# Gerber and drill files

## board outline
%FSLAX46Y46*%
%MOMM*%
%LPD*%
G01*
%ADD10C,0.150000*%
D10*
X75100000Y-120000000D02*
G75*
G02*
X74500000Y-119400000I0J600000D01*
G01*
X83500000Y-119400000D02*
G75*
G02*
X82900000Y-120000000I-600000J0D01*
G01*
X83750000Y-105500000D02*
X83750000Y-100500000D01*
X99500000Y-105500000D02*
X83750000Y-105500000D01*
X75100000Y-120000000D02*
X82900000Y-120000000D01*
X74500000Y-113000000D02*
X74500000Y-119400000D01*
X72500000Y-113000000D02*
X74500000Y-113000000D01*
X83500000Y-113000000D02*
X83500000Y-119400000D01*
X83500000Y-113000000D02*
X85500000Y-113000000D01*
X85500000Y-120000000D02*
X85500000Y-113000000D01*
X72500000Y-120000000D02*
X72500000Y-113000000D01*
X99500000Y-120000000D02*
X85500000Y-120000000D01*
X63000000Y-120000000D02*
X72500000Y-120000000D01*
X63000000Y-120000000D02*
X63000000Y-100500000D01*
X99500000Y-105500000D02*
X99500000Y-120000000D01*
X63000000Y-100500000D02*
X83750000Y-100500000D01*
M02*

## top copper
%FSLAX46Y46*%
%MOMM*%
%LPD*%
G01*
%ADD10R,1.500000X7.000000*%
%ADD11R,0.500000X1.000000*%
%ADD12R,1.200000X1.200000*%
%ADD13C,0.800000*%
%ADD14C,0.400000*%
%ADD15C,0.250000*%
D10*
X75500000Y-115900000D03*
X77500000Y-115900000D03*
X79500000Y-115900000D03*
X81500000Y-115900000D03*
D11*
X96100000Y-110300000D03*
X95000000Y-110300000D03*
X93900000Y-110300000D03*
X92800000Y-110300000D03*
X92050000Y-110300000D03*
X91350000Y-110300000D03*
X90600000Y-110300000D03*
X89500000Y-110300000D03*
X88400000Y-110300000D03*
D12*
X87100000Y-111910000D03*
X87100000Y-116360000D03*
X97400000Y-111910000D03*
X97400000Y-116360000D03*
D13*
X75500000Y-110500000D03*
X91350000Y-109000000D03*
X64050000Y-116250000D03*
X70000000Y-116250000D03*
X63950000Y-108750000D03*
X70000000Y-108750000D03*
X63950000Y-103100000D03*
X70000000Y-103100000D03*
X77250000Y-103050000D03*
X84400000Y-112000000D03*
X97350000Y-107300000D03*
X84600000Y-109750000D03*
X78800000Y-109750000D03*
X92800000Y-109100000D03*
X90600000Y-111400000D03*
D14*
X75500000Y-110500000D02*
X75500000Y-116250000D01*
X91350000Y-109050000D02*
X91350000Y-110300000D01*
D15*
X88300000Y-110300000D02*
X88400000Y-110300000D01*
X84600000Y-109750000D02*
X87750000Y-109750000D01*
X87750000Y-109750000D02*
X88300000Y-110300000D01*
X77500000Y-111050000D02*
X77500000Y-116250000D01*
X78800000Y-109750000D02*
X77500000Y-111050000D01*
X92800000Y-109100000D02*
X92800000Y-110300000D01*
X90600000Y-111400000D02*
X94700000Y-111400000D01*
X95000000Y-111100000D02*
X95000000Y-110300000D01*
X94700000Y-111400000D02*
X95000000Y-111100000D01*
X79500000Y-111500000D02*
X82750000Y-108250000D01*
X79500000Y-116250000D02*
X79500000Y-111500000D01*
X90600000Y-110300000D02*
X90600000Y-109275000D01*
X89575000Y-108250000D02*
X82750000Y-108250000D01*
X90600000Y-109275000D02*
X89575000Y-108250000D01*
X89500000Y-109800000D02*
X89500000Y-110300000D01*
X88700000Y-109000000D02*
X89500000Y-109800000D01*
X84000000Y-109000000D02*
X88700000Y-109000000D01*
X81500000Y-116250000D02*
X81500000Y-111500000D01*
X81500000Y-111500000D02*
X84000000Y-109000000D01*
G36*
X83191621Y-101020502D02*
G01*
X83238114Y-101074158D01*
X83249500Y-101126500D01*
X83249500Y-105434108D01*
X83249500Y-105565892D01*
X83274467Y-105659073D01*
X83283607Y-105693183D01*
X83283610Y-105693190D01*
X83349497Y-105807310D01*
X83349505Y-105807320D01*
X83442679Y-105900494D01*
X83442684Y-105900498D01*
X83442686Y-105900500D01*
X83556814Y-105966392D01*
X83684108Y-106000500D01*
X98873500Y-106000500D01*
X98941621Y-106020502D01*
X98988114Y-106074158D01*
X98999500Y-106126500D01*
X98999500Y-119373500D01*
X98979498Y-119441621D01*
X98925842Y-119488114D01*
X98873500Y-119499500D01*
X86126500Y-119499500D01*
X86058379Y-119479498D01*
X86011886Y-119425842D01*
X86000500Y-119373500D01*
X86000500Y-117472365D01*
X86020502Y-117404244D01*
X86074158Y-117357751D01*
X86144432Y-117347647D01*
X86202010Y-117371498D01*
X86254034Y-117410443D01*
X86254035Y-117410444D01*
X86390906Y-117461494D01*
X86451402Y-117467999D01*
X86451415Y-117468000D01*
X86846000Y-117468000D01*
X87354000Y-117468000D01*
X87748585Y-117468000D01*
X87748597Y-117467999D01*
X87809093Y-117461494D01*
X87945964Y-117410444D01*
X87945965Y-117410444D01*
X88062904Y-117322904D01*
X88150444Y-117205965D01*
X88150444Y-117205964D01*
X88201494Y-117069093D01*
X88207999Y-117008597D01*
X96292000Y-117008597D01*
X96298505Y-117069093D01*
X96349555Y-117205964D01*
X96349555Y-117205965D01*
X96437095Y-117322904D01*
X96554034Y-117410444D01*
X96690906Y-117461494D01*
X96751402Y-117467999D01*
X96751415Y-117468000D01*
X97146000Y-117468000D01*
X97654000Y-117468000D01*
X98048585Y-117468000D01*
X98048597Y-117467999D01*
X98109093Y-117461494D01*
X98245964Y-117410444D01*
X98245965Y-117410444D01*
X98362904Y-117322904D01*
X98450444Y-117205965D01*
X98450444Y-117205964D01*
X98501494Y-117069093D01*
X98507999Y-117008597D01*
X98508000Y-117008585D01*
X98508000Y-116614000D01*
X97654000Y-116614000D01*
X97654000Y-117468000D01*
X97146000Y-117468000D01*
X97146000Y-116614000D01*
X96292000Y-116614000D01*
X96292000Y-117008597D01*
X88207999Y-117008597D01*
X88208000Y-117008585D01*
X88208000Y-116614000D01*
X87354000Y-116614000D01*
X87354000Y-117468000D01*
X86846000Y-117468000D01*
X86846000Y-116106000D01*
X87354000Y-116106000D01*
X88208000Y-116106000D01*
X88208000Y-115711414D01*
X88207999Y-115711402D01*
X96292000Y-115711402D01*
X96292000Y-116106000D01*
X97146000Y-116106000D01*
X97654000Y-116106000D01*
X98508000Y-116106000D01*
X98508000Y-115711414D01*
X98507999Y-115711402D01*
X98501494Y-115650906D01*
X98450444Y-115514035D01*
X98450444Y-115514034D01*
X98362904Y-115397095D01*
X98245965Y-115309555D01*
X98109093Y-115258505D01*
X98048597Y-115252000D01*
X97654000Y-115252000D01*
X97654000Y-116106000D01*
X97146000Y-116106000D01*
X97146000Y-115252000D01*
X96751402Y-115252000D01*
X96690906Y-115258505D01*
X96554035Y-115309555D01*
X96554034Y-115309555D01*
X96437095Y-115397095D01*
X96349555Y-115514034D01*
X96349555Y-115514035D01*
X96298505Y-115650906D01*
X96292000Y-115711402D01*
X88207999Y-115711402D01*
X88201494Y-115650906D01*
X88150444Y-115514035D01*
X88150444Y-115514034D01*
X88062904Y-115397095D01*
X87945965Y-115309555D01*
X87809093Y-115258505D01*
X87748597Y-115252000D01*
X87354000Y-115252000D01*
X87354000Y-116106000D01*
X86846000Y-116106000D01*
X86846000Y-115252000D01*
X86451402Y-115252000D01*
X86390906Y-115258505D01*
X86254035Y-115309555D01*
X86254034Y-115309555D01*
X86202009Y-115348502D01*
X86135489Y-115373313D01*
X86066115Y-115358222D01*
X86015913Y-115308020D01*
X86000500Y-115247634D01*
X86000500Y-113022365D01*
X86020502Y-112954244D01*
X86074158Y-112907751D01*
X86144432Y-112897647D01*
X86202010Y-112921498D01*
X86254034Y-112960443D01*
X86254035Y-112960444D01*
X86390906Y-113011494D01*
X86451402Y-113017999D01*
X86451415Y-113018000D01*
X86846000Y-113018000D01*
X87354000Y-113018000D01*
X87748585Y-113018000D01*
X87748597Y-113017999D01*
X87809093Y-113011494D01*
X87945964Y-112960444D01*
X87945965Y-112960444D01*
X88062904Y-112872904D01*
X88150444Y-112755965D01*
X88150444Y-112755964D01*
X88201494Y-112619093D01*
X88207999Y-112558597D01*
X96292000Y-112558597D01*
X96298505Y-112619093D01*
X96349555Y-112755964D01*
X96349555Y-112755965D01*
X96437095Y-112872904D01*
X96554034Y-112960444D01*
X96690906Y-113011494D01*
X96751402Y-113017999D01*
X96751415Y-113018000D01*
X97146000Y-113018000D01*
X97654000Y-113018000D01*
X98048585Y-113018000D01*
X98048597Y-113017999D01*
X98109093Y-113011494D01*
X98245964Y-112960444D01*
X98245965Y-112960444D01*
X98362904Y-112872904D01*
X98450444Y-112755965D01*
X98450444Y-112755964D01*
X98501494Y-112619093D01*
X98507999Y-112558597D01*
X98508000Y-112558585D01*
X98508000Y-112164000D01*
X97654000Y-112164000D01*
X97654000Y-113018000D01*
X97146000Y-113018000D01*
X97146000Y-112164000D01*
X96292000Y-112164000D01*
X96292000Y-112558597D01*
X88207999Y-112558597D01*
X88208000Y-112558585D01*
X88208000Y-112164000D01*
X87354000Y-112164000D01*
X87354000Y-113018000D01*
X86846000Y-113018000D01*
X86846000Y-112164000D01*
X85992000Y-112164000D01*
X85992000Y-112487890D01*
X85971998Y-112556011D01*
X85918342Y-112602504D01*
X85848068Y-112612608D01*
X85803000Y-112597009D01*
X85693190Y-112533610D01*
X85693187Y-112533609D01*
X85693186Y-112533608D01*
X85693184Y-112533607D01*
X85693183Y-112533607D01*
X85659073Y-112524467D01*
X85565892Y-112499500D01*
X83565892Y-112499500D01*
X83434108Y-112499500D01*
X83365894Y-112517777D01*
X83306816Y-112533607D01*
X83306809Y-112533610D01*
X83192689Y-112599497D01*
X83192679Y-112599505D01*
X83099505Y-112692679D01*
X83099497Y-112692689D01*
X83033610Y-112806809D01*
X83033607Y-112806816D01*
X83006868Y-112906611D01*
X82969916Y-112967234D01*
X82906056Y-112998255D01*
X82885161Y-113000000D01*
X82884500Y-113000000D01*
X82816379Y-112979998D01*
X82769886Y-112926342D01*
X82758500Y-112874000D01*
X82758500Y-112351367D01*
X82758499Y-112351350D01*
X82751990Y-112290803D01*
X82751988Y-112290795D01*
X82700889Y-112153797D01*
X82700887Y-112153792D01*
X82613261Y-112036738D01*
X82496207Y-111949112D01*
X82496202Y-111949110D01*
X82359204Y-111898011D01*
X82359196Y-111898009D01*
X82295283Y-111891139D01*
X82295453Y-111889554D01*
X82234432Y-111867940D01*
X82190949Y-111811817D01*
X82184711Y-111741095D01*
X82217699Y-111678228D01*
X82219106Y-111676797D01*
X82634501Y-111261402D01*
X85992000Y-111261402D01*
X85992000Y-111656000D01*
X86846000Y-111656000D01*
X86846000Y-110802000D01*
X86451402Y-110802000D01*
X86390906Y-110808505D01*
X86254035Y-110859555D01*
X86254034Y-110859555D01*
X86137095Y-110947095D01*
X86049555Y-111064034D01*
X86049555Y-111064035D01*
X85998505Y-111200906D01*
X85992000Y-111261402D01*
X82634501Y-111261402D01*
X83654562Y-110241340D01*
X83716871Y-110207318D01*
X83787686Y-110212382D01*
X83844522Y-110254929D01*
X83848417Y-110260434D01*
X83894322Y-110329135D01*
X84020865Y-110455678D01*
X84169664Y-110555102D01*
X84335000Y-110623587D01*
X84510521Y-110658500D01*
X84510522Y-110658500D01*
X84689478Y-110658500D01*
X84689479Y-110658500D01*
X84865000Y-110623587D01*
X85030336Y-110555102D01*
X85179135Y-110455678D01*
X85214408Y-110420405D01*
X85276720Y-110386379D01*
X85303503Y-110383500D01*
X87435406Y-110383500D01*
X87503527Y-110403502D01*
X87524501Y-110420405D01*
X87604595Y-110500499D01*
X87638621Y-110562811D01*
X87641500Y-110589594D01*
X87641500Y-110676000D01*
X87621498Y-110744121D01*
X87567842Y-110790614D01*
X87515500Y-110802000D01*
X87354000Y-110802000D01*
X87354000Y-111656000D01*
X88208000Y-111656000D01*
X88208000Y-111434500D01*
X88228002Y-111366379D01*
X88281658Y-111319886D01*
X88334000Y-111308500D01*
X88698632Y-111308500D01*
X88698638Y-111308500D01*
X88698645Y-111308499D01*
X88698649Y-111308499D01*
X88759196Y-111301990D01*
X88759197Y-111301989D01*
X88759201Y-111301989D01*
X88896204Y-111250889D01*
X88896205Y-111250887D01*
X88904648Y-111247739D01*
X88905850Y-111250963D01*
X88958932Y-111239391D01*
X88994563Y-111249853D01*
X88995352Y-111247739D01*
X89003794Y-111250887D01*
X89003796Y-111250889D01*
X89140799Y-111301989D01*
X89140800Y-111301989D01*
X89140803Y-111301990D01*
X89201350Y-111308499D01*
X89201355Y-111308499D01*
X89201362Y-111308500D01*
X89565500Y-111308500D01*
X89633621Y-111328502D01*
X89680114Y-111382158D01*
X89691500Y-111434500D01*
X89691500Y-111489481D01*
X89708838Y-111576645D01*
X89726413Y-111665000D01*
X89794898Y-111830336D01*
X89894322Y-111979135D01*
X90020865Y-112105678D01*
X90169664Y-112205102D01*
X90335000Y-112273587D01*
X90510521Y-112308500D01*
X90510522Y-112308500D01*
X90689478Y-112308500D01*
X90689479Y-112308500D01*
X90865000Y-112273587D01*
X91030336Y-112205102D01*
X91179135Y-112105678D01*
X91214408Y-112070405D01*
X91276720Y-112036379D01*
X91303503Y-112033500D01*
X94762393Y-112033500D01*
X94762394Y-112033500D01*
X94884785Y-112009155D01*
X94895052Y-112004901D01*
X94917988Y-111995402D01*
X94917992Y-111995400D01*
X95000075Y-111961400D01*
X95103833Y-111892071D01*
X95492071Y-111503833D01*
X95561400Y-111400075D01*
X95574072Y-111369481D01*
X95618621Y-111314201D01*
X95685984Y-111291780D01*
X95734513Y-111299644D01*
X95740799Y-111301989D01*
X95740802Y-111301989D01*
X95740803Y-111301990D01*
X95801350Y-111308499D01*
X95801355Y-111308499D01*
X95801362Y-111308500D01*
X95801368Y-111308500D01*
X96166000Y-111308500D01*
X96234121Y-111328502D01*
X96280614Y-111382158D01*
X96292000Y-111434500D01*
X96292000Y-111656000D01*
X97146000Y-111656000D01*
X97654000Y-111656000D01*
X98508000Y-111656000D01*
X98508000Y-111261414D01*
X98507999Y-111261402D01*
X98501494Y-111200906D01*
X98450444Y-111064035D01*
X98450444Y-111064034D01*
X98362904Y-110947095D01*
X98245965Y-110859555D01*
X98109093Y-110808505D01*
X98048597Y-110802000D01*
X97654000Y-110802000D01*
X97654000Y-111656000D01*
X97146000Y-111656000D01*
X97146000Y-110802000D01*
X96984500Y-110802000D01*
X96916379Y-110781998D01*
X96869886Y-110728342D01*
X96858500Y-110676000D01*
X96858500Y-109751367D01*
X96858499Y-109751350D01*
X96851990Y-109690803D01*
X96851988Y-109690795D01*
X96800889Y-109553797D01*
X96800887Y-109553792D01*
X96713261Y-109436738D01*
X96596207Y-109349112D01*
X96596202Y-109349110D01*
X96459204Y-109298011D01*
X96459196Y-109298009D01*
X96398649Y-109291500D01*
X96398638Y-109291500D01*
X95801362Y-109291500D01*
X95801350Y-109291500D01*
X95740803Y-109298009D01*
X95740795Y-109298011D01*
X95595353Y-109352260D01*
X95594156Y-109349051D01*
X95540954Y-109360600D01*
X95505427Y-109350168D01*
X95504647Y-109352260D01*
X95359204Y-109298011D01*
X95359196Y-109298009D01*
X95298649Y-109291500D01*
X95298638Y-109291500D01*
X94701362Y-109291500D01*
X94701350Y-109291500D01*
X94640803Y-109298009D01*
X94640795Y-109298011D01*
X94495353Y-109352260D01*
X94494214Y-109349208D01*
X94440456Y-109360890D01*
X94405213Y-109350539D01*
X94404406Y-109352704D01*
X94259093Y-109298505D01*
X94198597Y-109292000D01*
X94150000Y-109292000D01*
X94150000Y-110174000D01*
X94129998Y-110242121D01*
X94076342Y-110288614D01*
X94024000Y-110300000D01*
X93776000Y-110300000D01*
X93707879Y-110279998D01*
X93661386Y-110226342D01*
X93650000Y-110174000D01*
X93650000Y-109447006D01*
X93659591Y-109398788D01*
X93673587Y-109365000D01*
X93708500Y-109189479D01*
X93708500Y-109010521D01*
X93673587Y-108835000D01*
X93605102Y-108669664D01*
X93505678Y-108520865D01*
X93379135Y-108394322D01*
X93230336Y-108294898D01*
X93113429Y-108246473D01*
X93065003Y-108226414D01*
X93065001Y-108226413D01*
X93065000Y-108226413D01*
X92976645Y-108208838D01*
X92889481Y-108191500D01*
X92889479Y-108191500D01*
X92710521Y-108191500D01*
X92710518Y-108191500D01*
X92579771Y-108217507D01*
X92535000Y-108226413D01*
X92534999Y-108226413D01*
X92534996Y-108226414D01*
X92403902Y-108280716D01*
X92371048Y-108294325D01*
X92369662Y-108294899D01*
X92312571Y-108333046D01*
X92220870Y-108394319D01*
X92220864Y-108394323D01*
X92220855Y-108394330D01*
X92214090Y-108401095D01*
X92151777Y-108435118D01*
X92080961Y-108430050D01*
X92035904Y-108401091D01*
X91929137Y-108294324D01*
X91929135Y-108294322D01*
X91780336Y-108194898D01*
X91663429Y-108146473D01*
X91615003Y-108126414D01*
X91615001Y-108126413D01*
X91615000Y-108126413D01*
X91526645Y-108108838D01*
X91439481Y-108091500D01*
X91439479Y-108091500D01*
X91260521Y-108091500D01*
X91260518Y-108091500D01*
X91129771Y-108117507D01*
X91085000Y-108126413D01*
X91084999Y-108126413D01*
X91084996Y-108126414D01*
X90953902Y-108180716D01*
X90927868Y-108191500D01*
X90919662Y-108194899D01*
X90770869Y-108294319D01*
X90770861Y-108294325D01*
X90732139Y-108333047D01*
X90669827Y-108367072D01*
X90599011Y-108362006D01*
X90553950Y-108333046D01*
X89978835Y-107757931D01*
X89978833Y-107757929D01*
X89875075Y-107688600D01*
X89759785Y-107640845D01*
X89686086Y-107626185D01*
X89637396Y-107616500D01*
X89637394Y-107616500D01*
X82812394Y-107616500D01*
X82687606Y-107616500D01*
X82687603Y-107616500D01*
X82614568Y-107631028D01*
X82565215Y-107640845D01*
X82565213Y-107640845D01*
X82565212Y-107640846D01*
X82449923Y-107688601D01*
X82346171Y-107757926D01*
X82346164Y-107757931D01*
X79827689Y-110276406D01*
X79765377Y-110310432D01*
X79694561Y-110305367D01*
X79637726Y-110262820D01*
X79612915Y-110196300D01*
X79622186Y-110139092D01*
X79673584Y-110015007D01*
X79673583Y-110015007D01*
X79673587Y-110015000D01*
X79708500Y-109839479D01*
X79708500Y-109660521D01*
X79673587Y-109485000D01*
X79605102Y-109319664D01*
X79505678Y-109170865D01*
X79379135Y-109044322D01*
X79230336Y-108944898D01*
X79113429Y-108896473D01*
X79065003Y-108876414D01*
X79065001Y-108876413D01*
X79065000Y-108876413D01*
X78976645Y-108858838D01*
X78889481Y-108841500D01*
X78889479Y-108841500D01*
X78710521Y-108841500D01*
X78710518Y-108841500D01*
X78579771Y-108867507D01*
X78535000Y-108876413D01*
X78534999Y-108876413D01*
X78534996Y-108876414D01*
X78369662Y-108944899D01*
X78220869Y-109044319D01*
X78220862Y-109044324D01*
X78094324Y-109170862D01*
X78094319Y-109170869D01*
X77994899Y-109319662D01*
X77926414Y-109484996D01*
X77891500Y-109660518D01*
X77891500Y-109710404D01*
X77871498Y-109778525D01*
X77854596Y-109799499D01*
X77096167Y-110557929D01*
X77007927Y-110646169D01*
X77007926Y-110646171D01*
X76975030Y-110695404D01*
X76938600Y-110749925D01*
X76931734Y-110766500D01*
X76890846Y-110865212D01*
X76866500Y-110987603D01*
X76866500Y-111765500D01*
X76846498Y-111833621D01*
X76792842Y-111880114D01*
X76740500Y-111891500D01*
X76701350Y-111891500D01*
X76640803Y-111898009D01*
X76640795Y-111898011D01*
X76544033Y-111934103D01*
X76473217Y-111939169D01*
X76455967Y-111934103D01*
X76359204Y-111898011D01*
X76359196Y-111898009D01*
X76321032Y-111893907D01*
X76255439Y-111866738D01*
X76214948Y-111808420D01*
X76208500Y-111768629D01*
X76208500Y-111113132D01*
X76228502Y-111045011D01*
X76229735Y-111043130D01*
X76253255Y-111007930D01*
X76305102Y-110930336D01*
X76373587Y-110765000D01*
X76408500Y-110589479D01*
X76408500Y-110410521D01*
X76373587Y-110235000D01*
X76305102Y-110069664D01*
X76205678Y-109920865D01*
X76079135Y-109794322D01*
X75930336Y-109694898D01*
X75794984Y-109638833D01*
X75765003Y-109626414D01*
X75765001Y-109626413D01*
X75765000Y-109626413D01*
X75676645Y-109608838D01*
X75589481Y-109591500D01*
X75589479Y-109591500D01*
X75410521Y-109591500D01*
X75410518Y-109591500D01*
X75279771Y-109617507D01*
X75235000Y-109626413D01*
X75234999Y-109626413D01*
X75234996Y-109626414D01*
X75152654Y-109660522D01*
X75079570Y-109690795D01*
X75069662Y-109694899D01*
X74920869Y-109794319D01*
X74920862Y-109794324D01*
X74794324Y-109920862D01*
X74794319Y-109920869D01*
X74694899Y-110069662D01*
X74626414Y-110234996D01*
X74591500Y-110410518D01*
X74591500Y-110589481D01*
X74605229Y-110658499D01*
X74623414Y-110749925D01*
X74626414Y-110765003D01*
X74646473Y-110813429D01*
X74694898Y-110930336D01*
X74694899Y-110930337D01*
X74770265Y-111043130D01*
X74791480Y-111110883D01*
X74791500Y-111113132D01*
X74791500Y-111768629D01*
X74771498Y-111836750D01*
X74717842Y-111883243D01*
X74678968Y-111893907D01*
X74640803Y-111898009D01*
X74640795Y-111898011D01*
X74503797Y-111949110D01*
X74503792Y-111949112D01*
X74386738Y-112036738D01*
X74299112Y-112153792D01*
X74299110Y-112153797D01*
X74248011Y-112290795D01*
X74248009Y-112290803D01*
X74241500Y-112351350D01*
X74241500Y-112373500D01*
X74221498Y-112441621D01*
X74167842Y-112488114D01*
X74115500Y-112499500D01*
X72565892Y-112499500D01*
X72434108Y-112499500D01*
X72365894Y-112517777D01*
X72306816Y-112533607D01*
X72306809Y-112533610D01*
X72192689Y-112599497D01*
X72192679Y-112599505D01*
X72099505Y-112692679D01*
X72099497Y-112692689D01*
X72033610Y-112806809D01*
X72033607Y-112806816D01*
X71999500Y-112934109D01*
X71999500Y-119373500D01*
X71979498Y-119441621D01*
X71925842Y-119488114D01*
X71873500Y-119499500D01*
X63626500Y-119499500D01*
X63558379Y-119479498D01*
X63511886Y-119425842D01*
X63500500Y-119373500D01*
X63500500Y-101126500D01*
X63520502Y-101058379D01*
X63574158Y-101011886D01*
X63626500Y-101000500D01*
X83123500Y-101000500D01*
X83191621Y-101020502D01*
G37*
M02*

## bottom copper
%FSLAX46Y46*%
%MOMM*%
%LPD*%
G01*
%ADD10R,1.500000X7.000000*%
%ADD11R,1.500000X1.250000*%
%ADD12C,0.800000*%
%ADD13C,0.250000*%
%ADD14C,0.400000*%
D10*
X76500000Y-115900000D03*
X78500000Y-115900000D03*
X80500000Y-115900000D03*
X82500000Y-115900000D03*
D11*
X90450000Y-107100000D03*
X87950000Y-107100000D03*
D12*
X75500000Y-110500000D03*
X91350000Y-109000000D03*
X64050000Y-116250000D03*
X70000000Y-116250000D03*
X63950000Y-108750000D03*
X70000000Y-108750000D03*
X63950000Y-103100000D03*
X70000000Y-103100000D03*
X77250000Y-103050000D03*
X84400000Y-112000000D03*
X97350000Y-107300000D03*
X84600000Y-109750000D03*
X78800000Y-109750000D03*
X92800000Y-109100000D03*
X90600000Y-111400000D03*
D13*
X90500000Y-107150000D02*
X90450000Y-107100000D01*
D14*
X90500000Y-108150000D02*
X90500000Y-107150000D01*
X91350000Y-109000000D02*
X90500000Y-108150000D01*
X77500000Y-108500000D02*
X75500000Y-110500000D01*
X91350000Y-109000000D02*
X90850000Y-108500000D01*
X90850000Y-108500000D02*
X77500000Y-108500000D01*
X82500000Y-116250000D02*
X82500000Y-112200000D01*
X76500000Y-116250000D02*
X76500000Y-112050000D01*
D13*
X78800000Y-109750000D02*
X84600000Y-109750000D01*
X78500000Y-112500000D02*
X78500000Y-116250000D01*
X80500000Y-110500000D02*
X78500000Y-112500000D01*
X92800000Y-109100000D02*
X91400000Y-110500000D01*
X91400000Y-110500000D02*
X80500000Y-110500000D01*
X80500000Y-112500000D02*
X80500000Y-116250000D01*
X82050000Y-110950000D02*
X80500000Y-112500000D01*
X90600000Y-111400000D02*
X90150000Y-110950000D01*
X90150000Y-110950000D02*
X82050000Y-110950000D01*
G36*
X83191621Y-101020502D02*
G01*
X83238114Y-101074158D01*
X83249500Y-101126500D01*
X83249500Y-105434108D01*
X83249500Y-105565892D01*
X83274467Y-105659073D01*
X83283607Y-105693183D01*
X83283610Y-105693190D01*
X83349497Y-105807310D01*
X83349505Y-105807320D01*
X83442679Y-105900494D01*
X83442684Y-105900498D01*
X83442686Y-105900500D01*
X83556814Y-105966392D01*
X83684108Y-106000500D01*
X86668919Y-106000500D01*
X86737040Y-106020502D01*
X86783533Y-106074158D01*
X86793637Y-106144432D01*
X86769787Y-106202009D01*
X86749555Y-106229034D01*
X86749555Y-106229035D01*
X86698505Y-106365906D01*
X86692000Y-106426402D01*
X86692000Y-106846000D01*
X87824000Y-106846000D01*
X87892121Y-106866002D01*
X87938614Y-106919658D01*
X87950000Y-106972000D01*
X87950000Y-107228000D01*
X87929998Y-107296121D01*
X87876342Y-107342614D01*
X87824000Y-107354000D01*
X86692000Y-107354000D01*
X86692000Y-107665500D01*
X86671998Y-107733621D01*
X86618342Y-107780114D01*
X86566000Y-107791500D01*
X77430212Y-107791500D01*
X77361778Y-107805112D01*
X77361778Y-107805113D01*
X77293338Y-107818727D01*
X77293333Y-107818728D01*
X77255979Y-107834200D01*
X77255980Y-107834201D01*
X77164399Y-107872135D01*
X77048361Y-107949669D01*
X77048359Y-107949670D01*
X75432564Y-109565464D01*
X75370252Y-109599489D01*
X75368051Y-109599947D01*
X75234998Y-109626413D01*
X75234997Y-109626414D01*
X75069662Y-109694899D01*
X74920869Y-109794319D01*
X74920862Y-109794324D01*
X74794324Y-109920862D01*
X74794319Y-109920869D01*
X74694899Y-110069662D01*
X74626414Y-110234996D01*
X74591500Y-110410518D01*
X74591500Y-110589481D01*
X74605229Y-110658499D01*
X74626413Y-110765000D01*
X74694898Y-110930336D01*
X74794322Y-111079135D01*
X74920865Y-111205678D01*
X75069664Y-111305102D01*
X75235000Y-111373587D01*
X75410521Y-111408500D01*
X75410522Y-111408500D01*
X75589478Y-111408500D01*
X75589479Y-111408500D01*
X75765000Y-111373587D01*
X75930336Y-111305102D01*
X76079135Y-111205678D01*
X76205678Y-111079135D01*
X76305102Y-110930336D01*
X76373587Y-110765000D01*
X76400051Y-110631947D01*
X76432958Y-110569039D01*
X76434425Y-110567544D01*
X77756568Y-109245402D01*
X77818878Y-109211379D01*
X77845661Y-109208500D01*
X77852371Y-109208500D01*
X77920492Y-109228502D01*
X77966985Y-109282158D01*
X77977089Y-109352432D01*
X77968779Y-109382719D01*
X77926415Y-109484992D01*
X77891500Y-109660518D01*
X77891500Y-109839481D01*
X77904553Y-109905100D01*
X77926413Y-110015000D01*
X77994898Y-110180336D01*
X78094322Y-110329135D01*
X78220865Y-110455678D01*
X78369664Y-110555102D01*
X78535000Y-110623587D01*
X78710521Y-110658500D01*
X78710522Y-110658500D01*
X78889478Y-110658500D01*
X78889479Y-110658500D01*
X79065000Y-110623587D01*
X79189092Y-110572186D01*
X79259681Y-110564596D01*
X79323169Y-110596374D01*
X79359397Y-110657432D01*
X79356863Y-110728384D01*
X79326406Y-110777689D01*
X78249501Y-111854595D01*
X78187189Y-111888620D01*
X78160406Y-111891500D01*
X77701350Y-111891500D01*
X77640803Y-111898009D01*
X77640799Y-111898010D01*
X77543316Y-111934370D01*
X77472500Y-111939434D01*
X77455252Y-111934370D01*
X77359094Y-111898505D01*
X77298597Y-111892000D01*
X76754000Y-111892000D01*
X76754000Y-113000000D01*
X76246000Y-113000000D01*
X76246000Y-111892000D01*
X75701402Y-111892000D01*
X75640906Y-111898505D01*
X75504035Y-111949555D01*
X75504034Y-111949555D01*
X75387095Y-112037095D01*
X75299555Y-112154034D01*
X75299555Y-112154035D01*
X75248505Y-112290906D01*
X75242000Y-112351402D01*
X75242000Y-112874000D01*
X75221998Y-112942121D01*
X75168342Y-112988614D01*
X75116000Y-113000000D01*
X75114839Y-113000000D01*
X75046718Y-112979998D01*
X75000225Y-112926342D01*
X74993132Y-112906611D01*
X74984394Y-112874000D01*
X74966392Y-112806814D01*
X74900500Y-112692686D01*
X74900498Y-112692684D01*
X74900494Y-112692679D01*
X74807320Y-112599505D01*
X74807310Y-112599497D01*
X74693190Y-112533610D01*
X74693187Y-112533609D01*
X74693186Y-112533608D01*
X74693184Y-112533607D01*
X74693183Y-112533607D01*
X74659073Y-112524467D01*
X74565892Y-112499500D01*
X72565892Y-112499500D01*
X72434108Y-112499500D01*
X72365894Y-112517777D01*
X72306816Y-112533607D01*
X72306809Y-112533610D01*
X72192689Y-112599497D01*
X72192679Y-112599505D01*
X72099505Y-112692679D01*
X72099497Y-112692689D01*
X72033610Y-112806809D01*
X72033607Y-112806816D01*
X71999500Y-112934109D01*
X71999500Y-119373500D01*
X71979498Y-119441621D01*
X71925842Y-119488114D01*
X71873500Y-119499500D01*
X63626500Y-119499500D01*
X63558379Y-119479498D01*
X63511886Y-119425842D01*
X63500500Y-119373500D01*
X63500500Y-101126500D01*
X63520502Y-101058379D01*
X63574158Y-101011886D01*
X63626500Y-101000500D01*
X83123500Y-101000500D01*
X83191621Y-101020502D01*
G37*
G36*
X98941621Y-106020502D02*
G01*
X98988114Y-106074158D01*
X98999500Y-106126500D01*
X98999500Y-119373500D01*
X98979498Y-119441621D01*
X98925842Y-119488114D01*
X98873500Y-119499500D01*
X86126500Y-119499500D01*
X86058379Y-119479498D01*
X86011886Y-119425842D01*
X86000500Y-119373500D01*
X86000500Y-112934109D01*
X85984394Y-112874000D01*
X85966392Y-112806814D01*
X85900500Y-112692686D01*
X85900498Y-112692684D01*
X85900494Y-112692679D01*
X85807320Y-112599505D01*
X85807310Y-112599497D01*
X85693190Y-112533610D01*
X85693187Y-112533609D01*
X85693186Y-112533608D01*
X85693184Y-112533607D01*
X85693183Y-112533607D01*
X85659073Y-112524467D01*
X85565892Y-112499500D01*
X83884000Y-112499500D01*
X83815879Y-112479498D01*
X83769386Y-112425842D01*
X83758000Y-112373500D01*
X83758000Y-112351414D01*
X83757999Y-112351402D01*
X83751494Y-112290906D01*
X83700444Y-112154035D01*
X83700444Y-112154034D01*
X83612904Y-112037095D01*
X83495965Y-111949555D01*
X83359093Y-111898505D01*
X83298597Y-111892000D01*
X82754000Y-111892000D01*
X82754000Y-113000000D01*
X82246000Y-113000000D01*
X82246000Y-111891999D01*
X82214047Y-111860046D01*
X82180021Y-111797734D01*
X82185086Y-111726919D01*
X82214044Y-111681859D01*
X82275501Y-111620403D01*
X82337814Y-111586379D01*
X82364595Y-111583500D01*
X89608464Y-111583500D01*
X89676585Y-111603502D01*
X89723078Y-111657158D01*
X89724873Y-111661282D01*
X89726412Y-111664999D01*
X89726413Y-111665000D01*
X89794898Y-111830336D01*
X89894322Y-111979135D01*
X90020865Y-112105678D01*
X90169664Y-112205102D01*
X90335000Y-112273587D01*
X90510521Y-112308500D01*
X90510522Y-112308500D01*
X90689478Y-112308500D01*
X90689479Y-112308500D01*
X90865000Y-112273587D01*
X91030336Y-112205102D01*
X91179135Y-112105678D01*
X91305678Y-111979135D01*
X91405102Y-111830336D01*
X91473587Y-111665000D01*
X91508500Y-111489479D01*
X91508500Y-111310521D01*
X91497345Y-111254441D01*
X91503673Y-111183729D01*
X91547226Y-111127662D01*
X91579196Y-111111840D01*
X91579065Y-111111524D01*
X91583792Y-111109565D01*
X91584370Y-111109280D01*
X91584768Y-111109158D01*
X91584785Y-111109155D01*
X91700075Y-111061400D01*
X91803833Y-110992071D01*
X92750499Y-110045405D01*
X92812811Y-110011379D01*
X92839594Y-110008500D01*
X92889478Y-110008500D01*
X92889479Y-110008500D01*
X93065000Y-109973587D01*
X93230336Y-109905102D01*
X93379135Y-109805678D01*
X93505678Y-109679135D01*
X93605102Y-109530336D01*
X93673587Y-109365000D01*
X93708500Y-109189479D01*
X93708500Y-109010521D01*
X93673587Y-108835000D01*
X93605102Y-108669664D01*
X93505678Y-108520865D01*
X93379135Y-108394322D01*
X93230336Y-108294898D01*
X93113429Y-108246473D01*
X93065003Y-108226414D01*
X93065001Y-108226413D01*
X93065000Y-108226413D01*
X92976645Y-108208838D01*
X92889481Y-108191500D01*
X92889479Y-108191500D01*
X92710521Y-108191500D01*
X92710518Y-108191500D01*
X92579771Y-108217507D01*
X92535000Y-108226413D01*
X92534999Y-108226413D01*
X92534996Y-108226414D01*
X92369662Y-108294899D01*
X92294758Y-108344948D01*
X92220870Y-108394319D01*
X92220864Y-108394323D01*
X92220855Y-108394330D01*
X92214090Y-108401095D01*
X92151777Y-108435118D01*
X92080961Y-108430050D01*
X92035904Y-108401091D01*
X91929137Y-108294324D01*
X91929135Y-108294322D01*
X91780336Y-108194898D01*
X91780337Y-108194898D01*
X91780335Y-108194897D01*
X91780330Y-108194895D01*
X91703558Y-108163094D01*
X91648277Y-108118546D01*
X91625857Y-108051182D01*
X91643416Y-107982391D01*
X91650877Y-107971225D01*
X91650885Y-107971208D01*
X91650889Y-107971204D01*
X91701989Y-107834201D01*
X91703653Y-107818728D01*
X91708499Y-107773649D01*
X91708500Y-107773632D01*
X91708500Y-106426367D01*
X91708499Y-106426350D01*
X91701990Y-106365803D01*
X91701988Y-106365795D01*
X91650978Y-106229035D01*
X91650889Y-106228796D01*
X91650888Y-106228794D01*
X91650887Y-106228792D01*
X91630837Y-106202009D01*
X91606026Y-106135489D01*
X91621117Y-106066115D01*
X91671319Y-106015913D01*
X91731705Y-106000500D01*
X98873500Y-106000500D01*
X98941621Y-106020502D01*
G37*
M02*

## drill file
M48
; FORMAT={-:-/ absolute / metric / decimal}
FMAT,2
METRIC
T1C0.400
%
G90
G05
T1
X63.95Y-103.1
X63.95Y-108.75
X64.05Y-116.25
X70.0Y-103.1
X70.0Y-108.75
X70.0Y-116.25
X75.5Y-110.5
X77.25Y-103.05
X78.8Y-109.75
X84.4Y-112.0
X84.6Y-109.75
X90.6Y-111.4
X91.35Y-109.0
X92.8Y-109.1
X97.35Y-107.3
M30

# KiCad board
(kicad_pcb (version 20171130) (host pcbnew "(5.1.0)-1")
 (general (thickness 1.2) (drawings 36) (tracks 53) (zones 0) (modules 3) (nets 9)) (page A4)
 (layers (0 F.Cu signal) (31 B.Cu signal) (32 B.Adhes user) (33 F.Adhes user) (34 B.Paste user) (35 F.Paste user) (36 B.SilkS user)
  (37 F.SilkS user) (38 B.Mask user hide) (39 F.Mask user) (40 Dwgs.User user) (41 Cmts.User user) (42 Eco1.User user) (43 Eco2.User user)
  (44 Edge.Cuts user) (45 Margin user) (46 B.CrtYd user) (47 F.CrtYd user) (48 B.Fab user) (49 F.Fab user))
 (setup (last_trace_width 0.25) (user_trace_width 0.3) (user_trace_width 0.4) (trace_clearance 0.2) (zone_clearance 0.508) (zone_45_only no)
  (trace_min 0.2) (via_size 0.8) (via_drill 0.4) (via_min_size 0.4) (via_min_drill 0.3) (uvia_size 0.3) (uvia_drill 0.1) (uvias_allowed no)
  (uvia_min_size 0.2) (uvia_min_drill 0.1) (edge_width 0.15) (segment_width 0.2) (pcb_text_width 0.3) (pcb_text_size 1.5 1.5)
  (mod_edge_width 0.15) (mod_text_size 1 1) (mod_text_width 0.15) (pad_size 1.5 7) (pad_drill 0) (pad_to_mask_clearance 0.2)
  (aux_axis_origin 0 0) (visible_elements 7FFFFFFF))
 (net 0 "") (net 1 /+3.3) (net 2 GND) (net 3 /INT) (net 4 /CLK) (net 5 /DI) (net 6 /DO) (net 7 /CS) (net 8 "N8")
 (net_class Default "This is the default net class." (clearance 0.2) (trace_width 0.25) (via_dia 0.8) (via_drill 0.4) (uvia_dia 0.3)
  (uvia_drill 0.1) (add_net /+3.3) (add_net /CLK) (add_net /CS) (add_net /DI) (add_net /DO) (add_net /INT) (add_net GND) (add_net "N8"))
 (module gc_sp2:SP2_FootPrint (layer F.Cu) (at 75.5 115.9)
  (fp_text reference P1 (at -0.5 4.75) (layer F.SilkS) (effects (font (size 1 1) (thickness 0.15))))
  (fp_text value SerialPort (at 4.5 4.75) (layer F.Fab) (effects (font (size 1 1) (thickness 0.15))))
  (pad 1 smd rect (at 0 0) (size 1.5 7) (layers F.Cu F.Paste F.Mask) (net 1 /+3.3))
  (pad 2 smd rect (at 1 0) (size 1.5 7) (layers B.Cu B.Paste B.Mask) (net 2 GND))
  (pad 3 smd rect (at 2 0) (size 1.5 7) (layers F.Cu F.Paste F.Mask) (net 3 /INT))
  (pad 4 smd rect (at 3 0) (size 1.5 7) (layers B.Cu B.Adhes B.Mask) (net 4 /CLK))
  (pad 5 smd rect (at 4 0) (size 1.5 7) (layers F.Cu F.Paste F.Mask) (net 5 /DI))
  (pad 6 smd rect (at 5 0) (size 1.5 7) (layers B.Cu B.Paste B.Mask) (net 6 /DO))
  (pad 7 smd rect (at 6 0) (size 1.5 7) (layers F.Cu F.Paste F.Mask) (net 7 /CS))
  (pad 8 smd rect (at 7 0) (size 1.5 7) (layers B.Cu B.Paste B.Mask) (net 2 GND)))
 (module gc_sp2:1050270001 (layer F.Cu) (at 96.1 110.3 180)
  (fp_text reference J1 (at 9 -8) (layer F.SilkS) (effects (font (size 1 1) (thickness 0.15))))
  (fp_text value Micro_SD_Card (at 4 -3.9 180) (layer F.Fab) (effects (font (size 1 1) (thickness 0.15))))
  (pad 8 smd rect (at 0 0 180) (size 0.5 1) (layers F.Cu F.Paste F.Mask) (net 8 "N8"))
  (pad 7 smd rect (at 1.1 0 180) (size 0.5 1) (layers F.Cu F.Paste F.Mask) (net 6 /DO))
  (pad 6 smd rect (at 2.2 0 180) (size 0.5 1) (layers F.Cu F.Paste F.Mask) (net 2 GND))
  (pad 5 smd rect (at 3.3 0 180) (size 0.5 1) (layers F.Cu F.Paste F.Mask) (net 4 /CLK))
  (pad "" smd rect (at 4.05 0 180) (size 0.5 1) (layers F.Cu F.Paste F.Mask))
  (pad 4 smd rect (at 4.75 0 180) (size 0.5 1) (layers F.Cu F.Paste F.Mask) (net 1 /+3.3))
  (pad 3 smd rect (at 5.5 0 180) (size 0.5 1) (layers F.Cu F.Paste F.Mask) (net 5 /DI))
  (pad 2 smd rect (at 6.6 0 180) (size 0.5 1) (layers F.Cu F.Paste F.Mask) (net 7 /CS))
  (pad 1 smd rect (at 7.7 0 180) (size 0.5 1) (layers F.Cu F.Paste F.Mask) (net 3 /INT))
  (pad 9 smd rect (at 9 -1.61 180) (size 1.2 1.2) (layers F.Cu F.Paste F.Mask) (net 2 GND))
  (pad 9 smd rect (at 9 -6.06 180) (size 1.2 1.2) (layers F.Cu F.Paste F.Mask) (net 2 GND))
  (pad 9 smd rect (at -1.3 -1.61 180) (size 1.2 1.2) (layers F.Cu F.Paste F.Mask) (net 2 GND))
  (pad 9 smd rect (at -1.3 -6.06 180) (size 1.2 1.2) (layers F.Cu F.Paste F.Mask) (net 2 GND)))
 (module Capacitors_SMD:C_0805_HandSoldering (layer B.Cu) (at 89.2 107.1 180)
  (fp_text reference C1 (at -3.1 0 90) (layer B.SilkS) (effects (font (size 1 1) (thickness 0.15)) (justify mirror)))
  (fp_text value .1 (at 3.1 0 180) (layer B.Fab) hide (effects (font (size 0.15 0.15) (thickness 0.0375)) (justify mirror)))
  (pad 1 smd rect (at -1.25 0 180) (size 1.5 1.25) (layers B.Cu B.Paste B.Mask) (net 1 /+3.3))
  (pad 2 smd rect (at 1.25 0 180) (size 1.5 1.25) (layers B.Cu B.Paste B.Mask) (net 2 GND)))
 (gr_arc (start 75.1 119.4) (end 74.5 119.4) (angle -90) (layer Edge.Cuts) (width 0.15))
 (gr_arc (start 82.9 119.4) (end 82.9 120) (angle -90) (layer Edge.Cuts) (width 0.15))
 (gr_line (start 83.75 105.5) (end 83.75 100.5) (layer Edge.Cuts) (width 0.15))
 (gr_line (start 99.5 105.5) (end 83.75 105.5) (layer Edge.Cuts) (width 0.15))
 (gr_line (start 75.1 120) (end 82.9 120) (layer Edge.Cuts) (width 0.15))
 (gr_line (start 74.5 113) (end 74.5 119.4) (layer Edge.Cuts) (width 0.15))
 (gr_line (start 72.5 113) (end 74.5 113) (layer Edge.Cuts) (width 0.15))
 (gr_line (start 83.5 113) (end 83.5 119.4) (layer Edge.Cuts) (width 0.15))
 (gr_line (start 83.5 113) (end 85.5 113) (layer Edge.Cuts) (width 0.15))
 (gr_line (start 85.5 120) (end 85.5 113) (layer Edge.Cuts) (width 0.15))
 (gr_line (start 72.5 120) (end 72.5 113) (layer Edge.Cuts) (width 0.15))
 (gr_line (start 99.5 120) (end 85.5 120) (layer Edge.Cuts) (width 0.15))
 (gr_line (start 63 120) (end 72.5 120) (layer Edge.Cuts) (width 0.15))
 (gr_line (start 63 120) (end 63 100.5) (layer Edge.Cuts) (width 0.15))
 (gr_line (start 99.5 105.5) (end 99.5 120) (layer Edge.Cuts) (width 0.15))
 (gr_line (start 63 100.5) (end 83.75 100.5) (layer Edge.Cuts) (width 0.15))
 (via (at 75.5 110.5) (size 0.8) (drill 0.4) (layers F.Cu B.Cu) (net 1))
 (segment (start 75.5 110.5) (end 75.5 116.25) (width 0.4) (layer F.Cu) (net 1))
 (segment (start 90.5 107.15) (end 90.45 107.1) (width 0.25) (layer B.Cu) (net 1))
 (segment (start 91.35 109.05) (end 91.35 110.3) (width 0.4) (layer F.Cu) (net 1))
 (via (at 91.35 109) (size 0.8) (drill 0.4) (layers F.Cu B.Cu) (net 1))
 (segment (start 90.5 108.15) (end 90.5 107.15) (width 0.4) (layer B.Cu) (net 1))
 (segment (start 91.35 109) (end 90.5 108.15) (width 0.4) (layer B.Cu) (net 1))
 (segment (start 77.5 108.5) (end 75.5 110.5) (width 0.4) (layer B.Cu) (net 1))
 (segment (start 91.35 109) (end 90.85 108.5) (width 0.4) (layer B.Cu) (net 1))
 (segment (start 90.85 108.5) (end 77.5 108.5) (width 0.4) (layer B.Cu) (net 1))
 (via (at 64.05 116.25) (size 0.8) (drill 0.4) (layers F.Cu B.Cu) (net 2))
 (via (at 70 116.25) (size 0.8) (drill 0.4) (layers F.Cu B.Cu) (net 2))
 (via (at 63.95 108.75) (size 0.8) (drill 0.4) (layers F.Cu B.Cu) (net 2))
 (via (at 70 108.75) (size 0.8) (drill 0.4) (layers F.Cu B.Cu) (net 2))
 (via (at 63.95 103.1) (size 0.8) (drill 0.4) (layers F.Cu B.Cu) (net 2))
 (via (at 70 103.1) (size 0.8) (drill 0.4) (layers F.Cu B.Cu) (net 2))
 (via (at 77.25 103.05) (size 0.8) (drill 0.4) (layers F.Cu B.Cu) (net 2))
 (via (at 84.4 112) (size 0.8) (drill 0.4) (layers F.Cu B.Cu) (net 2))
 (via (at 97.35 107.3) (size 0.8) (drill 0.4) (layers F.Cu B.Cu) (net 2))
 (segment (start 82.5 116.25) (end 82.5 112.2) (width 0.4) (layer B.Cu) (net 2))
 (segment (start 76.5 116.25) (end 76.5 112.05) (width 0.4) (layer B.Cu) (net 2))
 (via (at 84.6 109.75) (size 0.8) (drill 0.4) (layers F.Cu B.Cu) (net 3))
 (segment (start 88.3 110.3) (end 88.4 110.3) (width 0.25) (layer F.Cu) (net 3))
 (segment (start 84.6 109.75) (end 87.75 109.75) (width 0.25) (layer F.Cu) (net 3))
 (segment (start 87.75 109.75) (end 88.3 110.3) (width 0.25) (layer F.Cu) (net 3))
 (via (at 78.8 109.75) (size 0.8) (drill 0.4) (layers F.Cu B.Cu) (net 3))
 (segment (start 78.8 109.75) (end 84.6 109.75) (width 0.25) (layer B.Cu) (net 3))
 (segment (start 77.5 111.05) (end 77.5 116.25) (width 0.25) (layer F.Cu) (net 3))
 (segment (start 78.8 109.75) (end 77.5 111.05) (width 0.25) (layer F.Cu) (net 3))
 (via (at 92.8 109.1) (size 0.8) (drill 0.4) (layers F.Cu B.Cu) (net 4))
 (segment (start 92.8 109.1) (end 92.8 110.3) (width 0.25) (layer F.Cu) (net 4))
 (segment (start 78.5 112.5) (end 78.5 116.25) (width 0.25) (layer B.Cu) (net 4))
 (segment (start 80.5 110.5) (end 78.5 112.5) (width 0.25) (layer B.Cu) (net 4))
 (segment (start 92.8 109.1) (end 91.4 110.5) (width 0.25) (layer B.Cu) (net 4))
 (segment (start 91.4 110.5) (end 80.5 110.5) (width 0.25) (layer B.Cu) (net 4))
 (via (at 90.6 111.4) (size 0.8) (drill 0.4) (layers F.Cu B.Cu) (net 6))
 (segment (start 80.5 112.5) (end 80.5 116.25) (width 0.25) (layer B.Cu) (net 6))
 (segment (start 82.05 110.95) (end 80.5 112.5) (width 0.25) (layer B.Cu) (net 6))
 (segment (start 90.6 111.4) (end 90.15 110.95) (width 0.25) (layer B.Cu) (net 6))
 (segment (start 90.15 110.95) (end 82.05 110.95) (width 0.25) (layer B.Cu) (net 6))
 (segment (start 90.6 111.4) (end 94.7 111.4) (width 0.25) (layer F.Cu) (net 6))
 (segment (start 95 111.1) (end 95 110.3) (width 0.25) (layer F.Cu) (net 6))
 (segment (start 94.7 111.4) (end 95 111.1) (width 0.25) (layer F.Cu) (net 6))
 (segment (start 79.5 111.5) (end 82.75 108.25) (width 0.25) (layer F.Cu) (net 5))
 (segment (start 79.5 116.25) (end 79.5 111.5) (width 0.25) (layer F.Cu) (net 5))
 (segment (start 90.6 110.3) (end 90.6 109.275) (width 0.25) (layer F.Cu) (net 5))
 (segment (start 89.575 108.25) (end 82.75 108.25) (width 0.25) (layer F.Cu) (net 5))
 (segment (start 90.6 109.275) (end 89.575 108.25) (width 0.25) (layer F.Cu) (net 5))
 (segment (start 89.5 109.8) (end 89.5 110.3) (width 0.25) (layer F.Cu) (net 7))
 (segment (start 88.7 109) (end 89.5 109.8) (width 0.25) (layer F.Cu) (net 7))
 (segment (start 84 109) (end 88.7 109) (width 0.25) (layer F.Cu) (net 7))
 (segment (start 81.5 116.25) (end 81.5 111.5) (width 0.25) (layer F.Cu) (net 7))
 (segment (start 81.5 111.5) (end 84 109) (width 0.25) (layer F.Cu) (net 7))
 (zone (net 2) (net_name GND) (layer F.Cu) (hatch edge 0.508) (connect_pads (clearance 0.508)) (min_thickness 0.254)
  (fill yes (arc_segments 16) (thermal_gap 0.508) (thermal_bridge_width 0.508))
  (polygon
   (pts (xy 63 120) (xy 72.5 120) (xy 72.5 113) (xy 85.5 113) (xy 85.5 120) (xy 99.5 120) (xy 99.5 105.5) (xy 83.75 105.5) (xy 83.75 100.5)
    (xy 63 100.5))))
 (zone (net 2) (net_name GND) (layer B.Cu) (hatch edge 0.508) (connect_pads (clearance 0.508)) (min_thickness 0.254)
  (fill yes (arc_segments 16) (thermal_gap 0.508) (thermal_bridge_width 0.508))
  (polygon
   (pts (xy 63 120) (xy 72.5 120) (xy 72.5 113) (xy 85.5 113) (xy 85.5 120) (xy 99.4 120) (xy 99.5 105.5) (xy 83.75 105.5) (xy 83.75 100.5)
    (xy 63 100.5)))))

